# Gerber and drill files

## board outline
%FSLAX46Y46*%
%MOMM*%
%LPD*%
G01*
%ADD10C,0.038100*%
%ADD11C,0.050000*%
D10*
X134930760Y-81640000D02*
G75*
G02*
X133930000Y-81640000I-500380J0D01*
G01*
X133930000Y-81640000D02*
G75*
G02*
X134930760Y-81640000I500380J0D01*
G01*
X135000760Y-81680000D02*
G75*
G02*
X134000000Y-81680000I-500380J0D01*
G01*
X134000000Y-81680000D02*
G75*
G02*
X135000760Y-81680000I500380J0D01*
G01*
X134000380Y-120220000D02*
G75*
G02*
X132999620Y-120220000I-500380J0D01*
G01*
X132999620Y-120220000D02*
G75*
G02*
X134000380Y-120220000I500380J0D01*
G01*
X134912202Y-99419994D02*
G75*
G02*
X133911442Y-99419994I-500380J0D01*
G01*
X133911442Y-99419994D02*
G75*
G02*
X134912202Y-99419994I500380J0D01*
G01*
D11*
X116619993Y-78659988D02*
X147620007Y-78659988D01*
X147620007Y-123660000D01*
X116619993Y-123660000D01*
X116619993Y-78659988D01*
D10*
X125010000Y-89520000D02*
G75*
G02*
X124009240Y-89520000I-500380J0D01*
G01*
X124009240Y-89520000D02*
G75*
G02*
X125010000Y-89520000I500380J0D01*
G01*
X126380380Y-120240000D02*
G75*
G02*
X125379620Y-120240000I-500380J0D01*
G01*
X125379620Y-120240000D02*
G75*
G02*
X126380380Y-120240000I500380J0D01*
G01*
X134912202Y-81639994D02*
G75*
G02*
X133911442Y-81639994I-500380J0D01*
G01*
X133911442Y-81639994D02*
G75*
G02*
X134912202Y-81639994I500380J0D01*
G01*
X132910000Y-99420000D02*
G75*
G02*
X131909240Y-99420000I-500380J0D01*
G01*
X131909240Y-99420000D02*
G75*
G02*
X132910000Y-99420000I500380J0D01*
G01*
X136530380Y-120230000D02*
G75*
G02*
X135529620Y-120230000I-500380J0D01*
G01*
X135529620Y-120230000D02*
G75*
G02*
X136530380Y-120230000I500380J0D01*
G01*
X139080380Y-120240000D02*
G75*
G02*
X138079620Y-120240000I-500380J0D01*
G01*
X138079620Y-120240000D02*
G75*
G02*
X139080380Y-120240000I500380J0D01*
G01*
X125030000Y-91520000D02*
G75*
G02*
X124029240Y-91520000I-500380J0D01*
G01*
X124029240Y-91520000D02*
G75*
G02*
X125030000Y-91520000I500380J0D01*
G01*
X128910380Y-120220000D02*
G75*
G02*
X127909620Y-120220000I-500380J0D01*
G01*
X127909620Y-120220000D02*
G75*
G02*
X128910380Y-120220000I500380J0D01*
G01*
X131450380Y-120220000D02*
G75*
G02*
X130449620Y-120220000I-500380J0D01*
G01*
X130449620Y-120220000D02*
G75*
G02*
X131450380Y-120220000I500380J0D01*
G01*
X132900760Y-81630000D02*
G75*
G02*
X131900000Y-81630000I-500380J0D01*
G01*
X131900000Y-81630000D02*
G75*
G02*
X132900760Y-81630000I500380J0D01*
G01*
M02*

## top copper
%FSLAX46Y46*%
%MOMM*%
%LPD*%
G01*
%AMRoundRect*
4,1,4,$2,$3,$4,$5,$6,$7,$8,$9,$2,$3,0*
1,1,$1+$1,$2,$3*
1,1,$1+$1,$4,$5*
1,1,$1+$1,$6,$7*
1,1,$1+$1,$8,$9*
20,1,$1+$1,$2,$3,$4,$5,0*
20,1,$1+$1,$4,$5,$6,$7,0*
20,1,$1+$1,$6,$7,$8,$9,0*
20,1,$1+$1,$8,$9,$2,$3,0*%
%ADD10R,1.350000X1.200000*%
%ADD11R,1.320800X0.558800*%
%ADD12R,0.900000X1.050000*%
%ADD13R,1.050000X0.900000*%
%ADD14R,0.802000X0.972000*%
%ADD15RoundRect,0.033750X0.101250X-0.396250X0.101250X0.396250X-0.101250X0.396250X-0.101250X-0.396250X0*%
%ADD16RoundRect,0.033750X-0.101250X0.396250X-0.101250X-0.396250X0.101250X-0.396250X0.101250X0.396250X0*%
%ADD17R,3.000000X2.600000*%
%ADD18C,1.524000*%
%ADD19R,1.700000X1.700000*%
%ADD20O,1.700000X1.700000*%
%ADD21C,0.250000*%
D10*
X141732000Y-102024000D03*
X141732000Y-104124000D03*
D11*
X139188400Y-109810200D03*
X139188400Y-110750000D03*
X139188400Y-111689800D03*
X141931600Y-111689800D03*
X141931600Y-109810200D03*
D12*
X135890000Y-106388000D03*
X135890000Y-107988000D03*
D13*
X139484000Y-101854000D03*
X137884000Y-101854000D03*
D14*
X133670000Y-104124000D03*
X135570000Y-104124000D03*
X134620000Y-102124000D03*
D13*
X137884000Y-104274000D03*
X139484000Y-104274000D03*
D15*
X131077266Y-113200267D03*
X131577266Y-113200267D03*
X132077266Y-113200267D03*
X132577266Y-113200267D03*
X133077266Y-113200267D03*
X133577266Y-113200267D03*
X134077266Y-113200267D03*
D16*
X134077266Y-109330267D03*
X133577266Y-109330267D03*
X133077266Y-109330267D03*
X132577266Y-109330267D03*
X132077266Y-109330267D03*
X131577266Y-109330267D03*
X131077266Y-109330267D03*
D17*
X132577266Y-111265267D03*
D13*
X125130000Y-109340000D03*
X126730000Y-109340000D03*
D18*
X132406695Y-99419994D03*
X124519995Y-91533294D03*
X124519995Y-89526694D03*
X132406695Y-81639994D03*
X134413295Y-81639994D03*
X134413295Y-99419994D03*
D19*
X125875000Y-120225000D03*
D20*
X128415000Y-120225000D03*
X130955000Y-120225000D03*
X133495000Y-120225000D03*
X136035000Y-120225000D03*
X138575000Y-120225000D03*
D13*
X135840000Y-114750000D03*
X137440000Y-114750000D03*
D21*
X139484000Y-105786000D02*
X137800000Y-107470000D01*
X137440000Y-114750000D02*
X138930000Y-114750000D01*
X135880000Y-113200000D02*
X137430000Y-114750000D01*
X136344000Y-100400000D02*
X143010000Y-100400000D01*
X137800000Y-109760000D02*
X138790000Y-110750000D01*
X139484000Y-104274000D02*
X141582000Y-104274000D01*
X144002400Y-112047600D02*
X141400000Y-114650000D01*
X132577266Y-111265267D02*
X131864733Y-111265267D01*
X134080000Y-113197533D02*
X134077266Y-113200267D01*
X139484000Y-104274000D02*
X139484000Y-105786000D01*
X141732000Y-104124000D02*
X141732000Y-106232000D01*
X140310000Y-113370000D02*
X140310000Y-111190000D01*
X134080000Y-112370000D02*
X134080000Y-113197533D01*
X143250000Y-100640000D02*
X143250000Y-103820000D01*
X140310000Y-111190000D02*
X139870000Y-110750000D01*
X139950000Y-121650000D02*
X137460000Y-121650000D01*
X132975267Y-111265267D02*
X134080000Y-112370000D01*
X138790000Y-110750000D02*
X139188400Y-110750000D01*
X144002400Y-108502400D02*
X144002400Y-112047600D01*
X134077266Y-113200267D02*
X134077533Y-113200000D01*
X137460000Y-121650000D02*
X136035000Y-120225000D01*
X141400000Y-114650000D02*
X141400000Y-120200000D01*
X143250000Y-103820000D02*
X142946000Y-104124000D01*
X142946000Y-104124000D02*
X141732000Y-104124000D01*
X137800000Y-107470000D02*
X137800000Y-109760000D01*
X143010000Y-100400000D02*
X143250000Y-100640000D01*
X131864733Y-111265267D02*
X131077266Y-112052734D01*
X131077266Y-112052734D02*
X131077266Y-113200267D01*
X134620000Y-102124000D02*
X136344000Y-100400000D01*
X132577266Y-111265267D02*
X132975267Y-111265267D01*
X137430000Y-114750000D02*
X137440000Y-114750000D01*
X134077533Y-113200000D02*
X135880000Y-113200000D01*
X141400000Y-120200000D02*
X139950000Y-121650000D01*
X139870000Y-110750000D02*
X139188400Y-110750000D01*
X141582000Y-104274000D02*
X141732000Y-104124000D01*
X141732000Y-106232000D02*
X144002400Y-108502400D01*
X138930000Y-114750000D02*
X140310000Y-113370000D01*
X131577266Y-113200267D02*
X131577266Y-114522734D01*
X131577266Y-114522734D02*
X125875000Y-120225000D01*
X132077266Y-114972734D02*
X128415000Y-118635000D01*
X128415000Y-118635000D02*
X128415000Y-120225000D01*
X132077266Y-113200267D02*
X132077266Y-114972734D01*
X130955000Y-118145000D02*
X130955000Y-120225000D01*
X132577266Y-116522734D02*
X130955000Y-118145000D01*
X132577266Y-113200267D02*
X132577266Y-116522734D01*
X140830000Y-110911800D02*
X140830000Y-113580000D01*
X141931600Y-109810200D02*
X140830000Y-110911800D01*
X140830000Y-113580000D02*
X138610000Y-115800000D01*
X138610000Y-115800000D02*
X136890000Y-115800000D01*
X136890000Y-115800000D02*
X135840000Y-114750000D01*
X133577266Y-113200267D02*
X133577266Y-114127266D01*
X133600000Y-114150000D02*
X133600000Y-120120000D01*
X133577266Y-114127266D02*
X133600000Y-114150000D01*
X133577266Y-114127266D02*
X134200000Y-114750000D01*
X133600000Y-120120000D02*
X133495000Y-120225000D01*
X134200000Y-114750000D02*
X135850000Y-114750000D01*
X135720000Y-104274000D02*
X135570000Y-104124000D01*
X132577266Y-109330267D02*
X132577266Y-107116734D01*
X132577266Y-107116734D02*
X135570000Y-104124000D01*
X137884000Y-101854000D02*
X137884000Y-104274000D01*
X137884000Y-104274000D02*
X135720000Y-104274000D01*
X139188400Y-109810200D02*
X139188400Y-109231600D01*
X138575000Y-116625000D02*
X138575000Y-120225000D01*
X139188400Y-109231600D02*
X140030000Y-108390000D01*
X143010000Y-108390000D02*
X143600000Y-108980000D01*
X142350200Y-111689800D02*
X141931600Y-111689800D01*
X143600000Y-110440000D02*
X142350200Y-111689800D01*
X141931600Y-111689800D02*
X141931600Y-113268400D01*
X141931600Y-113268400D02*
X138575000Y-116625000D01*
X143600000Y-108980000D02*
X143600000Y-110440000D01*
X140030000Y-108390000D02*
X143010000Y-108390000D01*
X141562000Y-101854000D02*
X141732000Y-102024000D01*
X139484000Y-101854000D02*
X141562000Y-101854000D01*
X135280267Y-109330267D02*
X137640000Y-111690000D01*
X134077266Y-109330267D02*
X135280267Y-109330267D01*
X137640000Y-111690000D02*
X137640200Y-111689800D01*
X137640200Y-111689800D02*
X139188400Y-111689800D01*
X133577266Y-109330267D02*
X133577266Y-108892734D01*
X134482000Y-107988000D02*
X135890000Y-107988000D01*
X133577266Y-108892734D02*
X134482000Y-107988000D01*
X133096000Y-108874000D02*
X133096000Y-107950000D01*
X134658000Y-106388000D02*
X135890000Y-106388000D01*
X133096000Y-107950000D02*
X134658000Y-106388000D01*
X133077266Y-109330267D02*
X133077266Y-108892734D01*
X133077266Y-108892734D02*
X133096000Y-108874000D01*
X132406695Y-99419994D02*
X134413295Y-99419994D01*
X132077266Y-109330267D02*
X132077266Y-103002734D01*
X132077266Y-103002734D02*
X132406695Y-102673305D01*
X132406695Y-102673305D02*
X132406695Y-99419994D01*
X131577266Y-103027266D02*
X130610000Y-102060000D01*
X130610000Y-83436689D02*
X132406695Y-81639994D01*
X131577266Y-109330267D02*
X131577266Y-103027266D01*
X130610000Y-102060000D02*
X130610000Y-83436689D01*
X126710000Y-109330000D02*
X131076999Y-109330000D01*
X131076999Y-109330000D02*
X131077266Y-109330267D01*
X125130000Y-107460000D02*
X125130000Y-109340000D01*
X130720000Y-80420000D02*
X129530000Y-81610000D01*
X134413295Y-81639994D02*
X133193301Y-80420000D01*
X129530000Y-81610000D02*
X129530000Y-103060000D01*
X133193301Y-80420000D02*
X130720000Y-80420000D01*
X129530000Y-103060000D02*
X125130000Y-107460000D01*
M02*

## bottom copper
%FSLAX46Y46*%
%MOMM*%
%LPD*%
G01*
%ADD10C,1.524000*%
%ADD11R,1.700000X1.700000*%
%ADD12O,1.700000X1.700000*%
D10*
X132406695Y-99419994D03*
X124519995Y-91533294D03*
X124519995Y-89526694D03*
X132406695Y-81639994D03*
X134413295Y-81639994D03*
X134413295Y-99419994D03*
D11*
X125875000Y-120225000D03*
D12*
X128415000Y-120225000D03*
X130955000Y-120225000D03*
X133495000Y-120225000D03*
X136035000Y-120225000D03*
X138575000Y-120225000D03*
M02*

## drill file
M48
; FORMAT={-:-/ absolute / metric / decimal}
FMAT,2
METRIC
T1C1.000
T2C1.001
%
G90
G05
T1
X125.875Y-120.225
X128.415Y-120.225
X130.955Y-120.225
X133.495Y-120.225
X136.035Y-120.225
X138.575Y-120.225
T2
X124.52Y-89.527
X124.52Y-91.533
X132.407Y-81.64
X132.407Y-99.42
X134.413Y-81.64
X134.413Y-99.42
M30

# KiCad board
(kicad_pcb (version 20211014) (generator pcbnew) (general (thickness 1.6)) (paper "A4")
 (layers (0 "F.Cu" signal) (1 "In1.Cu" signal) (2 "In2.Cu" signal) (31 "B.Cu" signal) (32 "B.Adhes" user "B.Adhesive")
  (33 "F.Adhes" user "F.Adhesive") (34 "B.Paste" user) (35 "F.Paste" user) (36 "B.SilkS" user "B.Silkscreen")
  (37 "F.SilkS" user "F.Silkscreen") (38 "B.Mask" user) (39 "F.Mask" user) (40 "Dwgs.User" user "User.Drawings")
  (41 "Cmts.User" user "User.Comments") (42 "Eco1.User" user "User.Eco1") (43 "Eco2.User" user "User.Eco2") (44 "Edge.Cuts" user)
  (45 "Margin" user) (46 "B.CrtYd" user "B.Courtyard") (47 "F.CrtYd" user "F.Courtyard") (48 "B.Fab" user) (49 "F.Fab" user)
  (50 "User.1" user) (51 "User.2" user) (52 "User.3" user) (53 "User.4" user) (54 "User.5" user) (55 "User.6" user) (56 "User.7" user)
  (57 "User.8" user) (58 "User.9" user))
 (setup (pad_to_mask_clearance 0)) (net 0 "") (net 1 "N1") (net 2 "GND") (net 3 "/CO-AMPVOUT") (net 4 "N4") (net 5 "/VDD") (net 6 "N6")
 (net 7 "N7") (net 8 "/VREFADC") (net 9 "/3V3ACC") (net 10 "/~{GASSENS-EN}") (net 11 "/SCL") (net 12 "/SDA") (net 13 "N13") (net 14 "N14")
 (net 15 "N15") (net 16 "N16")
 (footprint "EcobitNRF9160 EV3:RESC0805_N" (layer "F.Cu") (at 141.732 103.124 -90)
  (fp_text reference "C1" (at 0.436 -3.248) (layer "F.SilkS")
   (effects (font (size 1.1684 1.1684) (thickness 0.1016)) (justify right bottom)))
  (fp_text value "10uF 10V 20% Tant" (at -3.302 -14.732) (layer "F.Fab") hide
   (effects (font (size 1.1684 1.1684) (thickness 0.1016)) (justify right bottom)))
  (pad "1" smd rect (at -1.1 0 270) (size 1.2 1.35) (layers "F.Cu" "F.Paste" "F.Mask") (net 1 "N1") (solder_mask_margin 0.1016))
  (pad "2" smd rect (at 1 0 270) (size 1.2 1.35) (layers "F.Cu" "F.Paste" "F.Mask") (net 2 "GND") (solder_mask_margin 0.1016)))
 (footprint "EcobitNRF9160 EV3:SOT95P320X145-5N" (layer "F.Cu") (at 140.56 110.75)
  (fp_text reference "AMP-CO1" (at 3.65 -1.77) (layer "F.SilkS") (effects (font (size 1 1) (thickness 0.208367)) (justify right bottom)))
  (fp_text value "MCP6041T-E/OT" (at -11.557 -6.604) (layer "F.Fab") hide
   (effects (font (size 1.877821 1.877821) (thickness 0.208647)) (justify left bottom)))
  (pad "1" smd rect (at -1.3716 -0.9398) (size 1.3208 0.5588) (layers "F.Cu" "F.Paste" "F.Mask") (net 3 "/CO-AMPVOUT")
   (solder_mask_margin 0.1016))
  (pad "2" smd rect (at -1.3716 0) (size 1.3208 0.5588) (layers "F.Cu" "F.Paste" "F.Mask") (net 2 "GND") (solder_mask_margin 0.1016))
  (pad "3" smd rect (at -1.3716 0.9398) (size 1.3208 0.5588) (layers "F.Cu" "F.Paste" "F.Mask") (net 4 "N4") (solder_mask_margin 0.1016))
  (pad "4" smd rect (at 1.3716 0.9398) (size 1.3208 0.5588) (layers "F.Cu" "F.Paste" "F.Mask") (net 3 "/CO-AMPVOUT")
   (solder_mask_margin 0.1016))
  (pad "5" smd rect (at 1.3716 -0.9398) (size 1.3208 0.5588) (layers "F.Cu" "F.Paste" "F.Mask") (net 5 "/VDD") (solder_mask_margin 0.1016)))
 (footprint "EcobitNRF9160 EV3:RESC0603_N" (layer "F.Cu") (at 135.89 107.188 -90)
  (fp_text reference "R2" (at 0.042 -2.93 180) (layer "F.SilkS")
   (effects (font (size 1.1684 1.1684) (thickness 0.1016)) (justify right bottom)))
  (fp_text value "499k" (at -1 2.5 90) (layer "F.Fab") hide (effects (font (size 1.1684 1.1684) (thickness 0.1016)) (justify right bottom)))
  (pad "1" smd rect (at -0.8 0 270) (size 1.05 0.9) (layers "F.Cu" "F.Paste" "F.Mask") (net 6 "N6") (solder_mask_margin 0.1016))
  (pad "2" smd rect (at 0.8 0 270) (size 1.05 0.9) (layers "F.Cu" "F.Paste" "F.Mask") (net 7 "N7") (solder_mask_margin 0.1016)))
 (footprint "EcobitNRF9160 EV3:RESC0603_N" (layer "F.Cu") (at 138.684 101.854 180)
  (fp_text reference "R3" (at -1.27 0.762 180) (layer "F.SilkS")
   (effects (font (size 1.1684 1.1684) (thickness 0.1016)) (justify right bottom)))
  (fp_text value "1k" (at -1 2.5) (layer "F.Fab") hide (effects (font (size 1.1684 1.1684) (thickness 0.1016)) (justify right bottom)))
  (pad "1" smd rect (at -0.8 0 180) (size 1.05 0.9) (layers "F.Cu" "F.Paste" "F.Mask") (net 1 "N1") (solder_mask_margin 0.1016))
  (pad "2" smd rect (at 0.8 0 180) (size 1.05 0.9) (layers "F.Cu" "F.Paste" "F.Mask") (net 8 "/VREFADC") (solder_mask_margin 0.1016)))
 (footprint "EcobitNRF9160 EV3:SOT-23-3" (layer "F.Cu") (at 134.62 103.124)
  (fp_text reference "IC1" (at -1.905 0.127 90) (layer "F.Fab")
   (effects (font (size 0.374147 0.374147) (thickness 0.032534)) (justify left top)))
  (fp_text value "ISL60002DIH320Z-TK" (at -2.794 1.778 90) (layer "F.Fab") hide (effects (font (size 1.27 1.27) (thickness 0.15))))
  (pad "1" smd rect (at -0.95 1 90) (size 0.972 0.802) (layers "F.Cu" "F.Paste" "F.Mask") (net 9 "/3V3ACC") (solder_mask_margin 0.1016))
  (pad "2" smd rect (at 0.95 1 90) (size 0.972 0.802) (layers "F.Cu" "F.Paste" "F.Mask") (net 8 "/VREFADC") (solder_mask_margin 0.1016))
  (pad "3" smd rect (at 0 -1 90) (size 0.972 0.802) (layers "F.Cu" "F.Paste" "F.Mask") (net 2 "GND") (solder_mask_margin 0.1016)))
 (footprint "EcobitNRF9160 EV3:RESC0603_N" (layer "F.Cu") (at 138.684 104.274)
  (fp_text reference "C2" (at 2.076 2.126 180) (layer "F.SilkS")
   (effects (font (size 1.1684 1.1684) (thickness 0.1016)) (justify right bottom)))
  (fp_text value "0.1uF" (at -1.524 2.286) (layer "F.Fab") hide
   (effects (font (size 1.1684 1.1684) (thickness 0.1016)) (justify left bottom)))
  (pad "1" smd rect (at -0.8 0) (size 1.05 0.9) (layers "F.Cu" "F.Paste" "F.Mask") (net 8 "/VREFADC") (solder_mask_margin 0.1016))
  (pad "2" smd rect (at 0.8 0) (size 1.05 0.9) (layers "F.Cu" "F.Paste" "F.Mask") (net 2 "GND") (solder_mask_margin 0.1016)))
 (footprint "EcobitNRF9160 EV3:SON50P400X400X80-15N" (layer "F.Cu") (at 132.577266 111.265267 90)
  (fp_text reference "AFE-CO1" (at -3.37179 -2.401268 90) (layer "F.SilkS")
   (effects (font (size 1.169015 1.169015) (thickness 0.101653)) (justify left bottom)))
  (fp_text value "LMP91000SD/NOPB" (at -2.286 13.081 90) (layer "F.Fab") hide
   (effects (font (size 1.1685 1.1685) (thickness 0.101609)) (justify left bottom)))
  (pad "1" smd roundrect (at -1.935 -1.5 90) (size 0.86 0.27) (layers "F.Cu" "F.Paste" "F.Mask") (roundrect_rratio 0.125) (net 2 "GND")
   (solder_mask_margin 0.1016))
  (pad "2" smd roundrect (at -1.935 -1 90) (size 0.86 0.27) (layers "F.Cu" "F.Paste" "F.Mask") (roundrect_rratio 0.125)
   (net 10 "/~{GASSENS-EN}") (solder_mask_margin 0.1016))
  (pad "3" smd roundrect (at -1.935 -0.5 90) (size 0.86 0.27) (layers "F.Cu" "F.Paste" "F.Mask") (roundrect_rratio 0.125) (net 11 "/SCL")
   (solder_mask_margin 0.1016))
  (pad "4" smd roundrect (at -1.935 0 90) (size 0.86 0.27) (layers "F.Cu" "F.Paste" "F.Mask") (roundrect_rratio 0.125) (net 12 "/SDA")
   (solder_mask_margin 0.1016))
  (pad "5" smd roundrect (at -1.935 0.5 90) (size 0.86 0.27) (layers "F.Cu" "F.Paste" "F.Mask") (roundrect_rratio 0.125)
   (solder_mask_margin 0.1016))
  (pad "6" smd roundrect (at -1.935 1 90) (size 0.86 0.27) (layers "F.Cu" "F.Paste" "F.Mask") (roundrect_rratio 0.125) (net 5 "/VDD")
   (solder_mask_margin 0.1016))
  (pad "7" smd roundrect (at -1.935 1.5 90) (size 0.86 0.27) (layers "F.Cu" "F.Paste" "F.Mask") (roundrect_rratio 0.125) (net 2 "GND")
   (solder_mask_margin 0.1016))
  (pad "8" smd roundrect (at 1.935 1.5 270) (size 0.86 0.27) (layers "F.Cu" "F.Paste" "F.Mask") (roundrect_rratio 0.125) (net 4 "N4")
   (solder_mask_margin 0.1016))
  (pad "9" smd roundrect (at 1.935 1 270) (size 0.86 0.27) (layers "F.Cu" "F.Paste" "F.Mask") (roundrect_rratio 0.125) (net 7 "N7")
   (solder_mask_margin 0.1016))
  (pad "10" smd roundrect (at 1.935 0.5 270) (size 0.86 0.27) (layers "F.Cu" "F.Paste" "F.Mask") (roundrect_rratio 0.125) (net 6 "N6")
   (solder_mask_margin 0.1016))
  (pad "11" smd roundrect (at 1.935 0 270) (size 0.86 0.27) (layers "F.Cu" "F.Paste" "F.Mask") (roundrect_rratio 0.125) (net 8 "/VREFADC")
   (solder_mask_margin 0.1016))
  (pad "12" smd roundrect (at 1.935 -0.5 270) (size 0.86 0.27) (layers "F.Cu" "F.Paste" "F.Mask") (roundrect_rratio 0.125) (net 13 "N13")
   (solder_mask_margin 0.1016))
  (pad "13" smd roundrect (at 1.935 -1 270) (size 0.86 0.27) (layers "F.Cu" "F.Paste" "F.Mask") (roundrect_rratio 0.125) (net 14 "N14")
   (solder_mask_margin 0.1016))
  (pad "14" smd roundrect (at 1.935 -1.5 270) (size 0.86 0.27) (layers "F.Cu" "F.Paste" "F.Mask") (roundrect_rratio 0.125) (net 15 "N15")
   (solder_mask_margin 0.1016))
  (pad "15" smd rect (at 0 0 90) (size 2.6 3) (layers "F.Cu" "F.Mask") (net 2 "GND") (solder_mask_margin 0.1016)))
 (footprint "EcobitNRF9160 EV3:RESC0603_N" (layer "F.Cu") (at 125.93 109.34)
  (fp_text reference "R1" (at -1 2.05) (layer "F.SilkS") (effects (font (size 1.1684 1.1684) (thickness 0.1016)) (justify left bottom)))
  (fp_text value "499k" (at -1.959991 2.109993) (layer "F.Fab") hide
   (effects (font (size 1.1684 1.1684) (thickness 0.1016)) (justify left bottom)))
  (pad "1" smd rect (at -0.8 0) (size 1.05 0.9) (layers "F.Cu" "F.Paste" "F.Mask") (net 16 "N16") (solder_mask_margin 0.1016))
  (pad "2" smd rect (at 0.8 0) (size 1.05 0.9) (layers "F.Cu" "F.Paste" "F.Mask") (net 15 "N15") (solder_mask_margin 0.1016)))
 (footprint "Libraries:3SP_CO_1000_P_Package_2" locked (layer "F.Cu") (at 133.409995 90.529994)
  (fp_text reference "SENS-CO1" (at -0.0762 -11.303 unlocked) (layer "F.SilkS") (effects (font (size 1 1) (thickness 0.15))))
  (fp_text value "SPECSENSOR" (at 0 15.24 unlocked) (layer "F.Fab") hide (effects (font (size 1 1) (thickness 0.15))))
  (pad "1" thru_hole circle locked (at -1.0033 8.89) (size 1.524 1.524) (drill 1.00076) (layers *.Cu *.Mask) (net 13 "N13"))
  (pad "2" thru_hole circle locked (at -8.89 1.0033) (size 1.524 1.524) (drill 1.00076) (layers *.Cu *.Mask))
  (pad "3" thru_hole circle locked (at -8.89 -1.0033) (size 1.524 1.524) (drill 1.00076) (layers *.Cu *.Mask))
  (pad "4" thru_hole circle locked (at -1.0033 -8.89) (size 1.524 1.524) (drill 1.00076) (layers *.Cu *.Mask) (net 14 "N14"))
  (pad "5" thru_hole circle locked (at 1.0033 -8.89) (size 1.524 1.524) (drill 1.00076) (layers *.Cu *.Mask) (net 16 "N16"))
  (pad "6" thru_hole circle locked (at 1.0033 8.89) (size 1.524 1.524) (drill 1.00076) (layers *.Cu *.Mask) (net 13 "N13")))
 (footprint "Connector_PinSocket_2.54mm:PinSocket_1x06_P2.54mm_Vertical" (layer "F.Cu") (at 125.875 120.225 90)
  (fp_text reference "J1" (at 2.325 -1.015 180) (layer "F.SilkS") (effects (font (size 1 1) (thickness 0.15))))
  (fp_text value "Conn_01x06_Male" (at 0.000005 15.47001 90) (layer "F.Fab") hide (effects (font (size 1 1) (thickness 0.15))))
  (pad "1" thru_hole rect (at 0 0 90) (size 1.7 1.7) (drill 1) (layers *.Cu *.Mask) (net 10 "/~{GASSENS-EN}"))
  (pad "2" thru_hole oval (at 0 2.54 90) (size 1.7 1.7) (drill 1) (layers *.Cu *.Mask) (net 11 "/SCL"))
  (pad "3" thru_hole oval (at 0 5.08 90) (size 1.7 1.7) (drill 1) (layers *.Cu *.Mask) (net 12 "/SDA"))
  (pad "4" thru_hole oval (at 0 7.62 90) (size 1.7 1.7) (drill 1) (layers *.Cu *.Mask) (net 5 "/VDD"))
  (pad "5" thru_hole oval (at 0 10.16 90) (size 1.7 1.7) (drill 1) (layers *.Cu *.Mask) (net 2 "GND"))
  (pad "6" thru_hole oval (at 0 12.7 90) (size 1.7 1.7) (drill 1) (layers *.Cu *.Mask) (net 3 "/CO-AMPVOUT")))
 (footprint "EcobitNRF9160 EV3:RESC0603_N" (layer "F.Cu") (at 136.64 114.75)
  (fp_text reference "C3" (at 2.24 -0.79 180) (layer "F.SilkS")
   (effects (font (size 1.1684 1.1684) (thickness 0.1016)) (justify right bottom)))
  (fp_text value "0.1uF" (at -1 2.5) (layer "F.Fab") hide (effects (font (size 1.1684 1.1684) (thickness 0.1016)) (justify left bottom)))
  (pad "1" smd rect (at -0.8 0) (size 1.05 0.9) (layers "F.Cu" "F.Paste" "F.Mask") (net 5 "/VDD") (solder_mask_margin 0.1016))
  (pad "2" smd rect (at 0.8 0) (size 1.05 0.9) (layers "F.Cu" "F.Paste" "F.Mask") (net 2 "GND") (solder_mask_margin 0.1016)))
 (gr_circle (center 134.43038 81.64) (end 134.93076 81.64) (layer "Edge.Cuts") (width 0.0381) (fill none))
 (gr_circle (center 134.50038 81.68) (end 135.00076 81.68) (layer "Edge.Cuts") (width 0.0381) (fill none))
 (gr_circle (center 133.5 120.22) (end 134.00038 120.22) (layer "Edge.Cuts") (width 0.0381) (fill none))
 (gr_circle (center 134.411822 99.419994) (end 134.912202 99.419994) (layer "Edge.Cuts") (width 0.0381) (fill none))
 (gr_rect (start 116.619993 78.659988) (end 147.620007 123.66) (layer "Edge.Cuts") (width 0.05) (fill none))
 (gr_circle (center 124.50962 89.52) (end 125.01 89.52) (layer "Edge.Cuts") (width 0.0381) (fill none))
 (gr_circle (center 125.88 120.24) (end 126.38038 120.24) (layer "Edge.Cuts") (width 0.0381) (fill none))
 (gr_circle (center 134.411822 81.639994) (end 134.912202 81.639994) (layer "Edge.Cuts") (width 0.0381) (fill none))
 (gr_circle (center 132.40962 99.42) (end 132.91 99.42) (layer "Edge.Cuts") (width 0.0381) (fill none))
 (gr_circle (center 136.03 120.23) (end 136.53038 120.23) (layer "Edge.Cuts") (width 0.0381) (fill none))
 (gr_circle (center 138.58 120.24) (end 139.08038 120.24) (layer "Edge.Cuts") (width 0.0381) (fill none))
 (gr_circle (center 124.52962 91.52) (end 125.03 91.52) (layer "Edge.Cuts") (width 0.0381) (fill none))
 (gr_circle (center 128.41 120.22) (end 128.91038 120.22) (layer "Edge.Cuts") (width 0.0381) (fill none))
 (gr_circle (center 130.95 120.22) (end 131.45038 120.22) (layer "Edge.Cuts") (width 0.0381) (fill none))
 (gr_circle (center 132.40038 81.63) (end 132.90076 81.63) (layer "Edge.Cuts") (width 0.0381) (fill none))
 (segment (start 139.484 105.786) (end 137.8 107.47) (width 0.25) (layer "F.Cu") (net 2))
 (segment (start 137.44 114.75) (end 138.93 114.75) (width 0.25) (layer "F.Cu") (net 2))
 (segment (start 135.88 113.2) (end 137.43 114.75) (width 0.25) (layer "F.Cu") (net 2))
 (segment (start 136.344 100.4) (end 143.01 100.4) (width 0.25) (layer "F.Cu") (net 2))
 (segment (start 137.8 109.76) (end 138.79 110.75) (width 0.25) (layer "F.Cu") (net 2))
 (segment (start 139.484 104.274) (end 141.582 104.274) (width 0.25) (layer "F.Cu") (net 2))
 (segment (start 144.0024 112.0476) (end 141.4 114.65) (width 0.25) (layer "F.Cu") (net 2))
 (segment (start 132.577266 111.265267) (end 131.864733 111.265267) (width 0.25) (layer "F.Cu") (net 2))
 (segment (start 134.08 113.197533) (end 134.077266 113.200267) (width 0.25) (layer "F.Cu") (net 2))
 (segment (start 139.484 104.274) (end 139.484 105.786) (width 0.25) (layer "F.Cu") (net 2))
 (segment (start 141.732 104.124) (end 141.732 106.232) (width 0.25) (layer "F.Cu") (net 2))
 (segment (start 140.31 113.37) (end 140.31 111.19) (width 0.25) (layer "F.Cu") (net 2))
 (segment (start 134.08 112.37) (end 134.08 113.197533) (width 0.25) (layer "F.Cu") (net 2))
 (segment (start 143.25 100.64) (end 143.25 103.82) (width 0.25) (layer "F.Cu") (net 2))
 (segment (start 140.31 111.19) (end 139.87 110.75) (width 0.25) (layer "F.Cu") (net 2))
 (segment (start 139.95 121.65) (end 137.46 121.65) (width 0.25) (layer "F.Cu") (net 2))
 (segment (start 132.975267 111.265267) (end 134.08 112.37) (width 0.25) (layer "F.Cu") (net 2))
 (segment (start 138.79 110.75) (end 139.1884 110.75) (width 0.25) (layer "F.Cu") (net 2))
 (segment (start 144.0024 108.5024) (end 144.0024 112.0476) (width 0.25) (layer "F.Cu") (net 2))
 (segment (start 134.077266 113.200267) (end 134.077533 113.2) (width 0.25) (layer "F.Cu") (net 2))
 (segment (start 137.46 121.65) (end 136.035 120.225) (width 0.25) (layer "F.Cu") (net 2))
 (segment (start 141.4 114.65) (end 141.4 120.2) (width 0.25) (layer "F.Cu") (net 2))
 (segment (start 143.25 103.82) (end 142.946 104.124) (width 0.25) (layer "F.Cu") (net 2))
 (segment (start 142.946 104.124) (end 141.732 104.124) (width 0.25) (layer "F.Cu") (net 2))
 (segment (start 137.8 107.47) (end 137.8 109.76) (width 0.25) (layer "F.Cu") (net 2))
 (segment (start 143.01 100.4) (end 143.25 100.64) (width 0.25) (layer "F.Cu") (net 2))
 (segment (start 131.864733 111.265267) (end 131.077266 112.052734) (width 0.25) (layer "F.Cu") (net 2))
 (segment (start 131.077266 112.052734) (end 131.077266 113.200267) (width 0.25) (layer "F.Cu") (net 2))
 (segment (start 134.62 102.124) (end 136.344 100.4) (width 0.25) (layer "F.Cu") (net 2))
 (segment (start 132.577266 111.265267) (end 132.975267 111.265267) (width 0.25) (layer "F.Cu") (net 2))
 (segment (start 137.43 114.75) (end 137.44 114.75) (width 0.25) (layer "F.Cu") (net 2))
 (segment (start 134.077533 113.2) (end 135.88 113.2) (width 0.25) (layer "F.Cu") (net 2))
 (segment (start 141.4 120.2) (end 139.95 121.65) (width 0.25) (layer "F.Cu") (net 2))
 (segment (start 139.87 110.75) (end 139.1884 110.75) (width 0.25) (layer "F.Cu") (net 2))
 (segment (start 141.582 104.274) (end 141.732 104.124) (width 0.25) (layer "F.Cu") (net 2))
 (segment (start 141.732 106.232) (end 144.0024 108.5024) (width 0.25) (layer "F.Cu") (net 2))
 (segment (start 138.93 114.75) (end 140.31 113.37) (width 0.25) (layer "F.Cu") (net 2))
 (segment (start 131.577266 113.200267) (end 131.577266 114.522734) (width 0.25) (layer "F.Cu") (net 10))
 (segment (start 131.577266 114.522734) (end 125.875 120.225) (width 0.25) (layer "F.Cu") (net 10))
 (segment (start 132.077266 114.972734) (end 128.415 118.635) (width 0.25) (layer "F.Cu") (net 11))
 (segment (start 128.415 118.635) (end 128.415 120.225) (width 0.25) (layer "F.Cu") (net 11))
 (segment (start 132.077266 113.200267) (end 132.077266 114.972734) (width 0.25) (layer "F.Cu") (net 11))
 (segment (start 130.955 118.145) (end 130.955 120.225) (width 0.25) (layer "F.Cu") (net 12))
 (segment (start 132.577266 116.522734) (end 130.955 118.145) (width 0.25) (layer "F.Cu") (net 12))
 (segment (start 132.577266 113.200267) (end 132.577266 116.522734) (width 0.25) (layer "F.Cu") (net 12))
 (segment (start 140.83 110.9118) (end 140.83 113.58) (width 0.25) (layer "F.Cu") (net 5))
 (segment (start 141.9316 109.8102) (end 140.83 110.9118) (width 0.25) (layer "F.Cu") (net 5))
 (segment (start 140.83 113.58) (end 138.61 115.8) (width 0.25) (layer "F.Cu") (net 5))
 (segment (start 138.61 115.8) (end 136.89 115.8) (width 0.25) (layer "F.Cu") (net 5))
 (segment (start 136.89 115.8) (end 135.84 114.75) (width 0.25) (layer "F.Cu") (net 5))
 (segment (start 133.577266 113.200267) (end 133.577266 114.127266) (width 0.25) (layer "F.Cu") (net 5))
 (segment (start 133.6 114.15) (end 133.6 120.12) (width 0.25) (layer "F.Cu") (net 5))
 (segment (start 133.577266 114.127266) (end 133.6 114.15) (width 0.25) (layer "F.Cu") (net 5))
 (segment (start 133.577266 114.127266) (end 134.2 114.75) (width 0.25) (layer "F.Cu") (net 5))
 (segment (start 133.6 120.12) (end 133.495 120.225) (width 0.25) (layer "F.Cu") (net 5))
 (segment (start 134.2 114.75) (end 135.85 114.75) (width 0.25) (layer "F.Cu") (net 5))
 (segment (start 135.72 104.274) (end 135.57 104.124) (width 0.25) (layer "F.Cu") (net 8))
 (segment (start 132.577266 109.330267) (end 132.577266 107.116734) (width 0.25) (layer "F.Cu") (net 8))
 (segment (start 132.577266 107.116734) (end 135.57 104.124) (width 0.25) (layer "F.Cu") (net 8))
 (segment (start 137.884 101.854) (end 137.884 104.274) (width 0.25) (layer "F.Cu") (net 8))
 (segment (start 137.884 104.274) (end 135.72 104.274) (width 0.25) (layer "F.Cu") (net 8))
 (segment (start 139.1884 109.8102) (end 139.1884 109.2316) (width 0.25) (layer "F.Cu") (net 3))
 (segment (start 138.575 116.625) (end 138.575 120.225) (width 0.25) (layer "F.Cu") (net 3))
 (segment (start 139.1884 109.2316) (end 140.03 108.39) (width 0.25) (layer "F.Cu") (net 3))
 (segment (start 143.01 108.39) (end 143.6 108.98) (width 0.25) (layer "F.Cu") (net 3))
 (segment (start 142.3502 111.6898) (end 141.9316 111.6898) (width 0.25) (layer "F.Cu") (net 3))
 (segment (start 143.6 110.44) (end 142.3502 111.6898) (width 0.25) (layer "F.Cu") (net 3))
 (segment (start 141.9316 111.6898) (end 141.9316 113.2684) (width 0.25) (layer "F.Cu") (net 3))
 (segment (start 141.9316 113.2684) (end 138.575 116.625) (width 0.25) (layer "F.Cu") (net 3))
 (segment (start 143.6 108.98) (end 143.6 110.44) (width 0.25) (layer "F.Cu") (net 3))
 (segment (start 140.03 108.39) (end 143.01 108.39) (width 0.25) (layer "F.Cu") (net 3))
 (segment (start 141.562 101.854) (end 141.732 102.024) (width 0.25) (layer "F.Cu") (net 1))
 (segment (start 139.484 101.854) (end 141.562 101.854) (width 0.25) (layer "F.Cu") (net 1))
 (segment (start 135.280267 109.330267) (end 137.64 111.69) (width 0.25) (layer "F.Cu") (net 4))
 (segment (start 134.077266 109.330267) (end 135.280267 109.330267) (width 0.25) (layer "F.Cu") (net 4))
 (segment (start 137.64 111.69) (end 137.6402 111.6898) (width 0.25) (layer "F.Cu") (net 4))
 (segment (start 137.6402 111.6898) (end 139.1884 111.6898) (width 0.25) (layer "F.Cu") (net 4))
 (segment (start 133.577266 109.330267) (end 133.577266 108.892734) (width 0.25) (layer "F.Cu") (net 7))
 (segment (start 134.482 107.988) (end 135.89 107.988) (width 0.25) (layer "F.Cu") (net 7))
 (segment (start 133.577266 108.892734) (end 134.482 107.988) (width 0.25) (layer "F.Cu") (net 7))
 (segment (start 133.096 108.874) (end 133.096 107.95) (width 0.25) (layer "F.Cu") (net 6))
 (segment (start 134.658 106.388) (end 135.89 106.388) (width 0.25) (layer "F.Cu") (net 6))
 (segment (start 133.096 107.95) (end 134.658 106.388) (width 0.25) (layer "F.Cu") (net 6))
 (segment (start 133.077266 109.330267) (end 133.077266 108.892734) (width 0.25) (layer "F.Cu") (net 6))
 (segment (start 133.077266 108.892734) (end 133.096 108.874) (width 0.25) (layer "F.Cu") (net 6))
 (segment (start 132.406695 99.419994) (end 134.413295 99.419994) (width 0.25) (layer "F.Cu") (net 13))
 (segment (start 132.077266 109.330267) (end 132.077266 103.002734) (width 0.25) (layer "F.Cu") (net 13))
 (segment (start 132.077266 103.002734) (end 132.406695 102.673305) (width 0.25) (layer "F.Cu") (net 13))
 (segment (start 132.406695 102.673305) (end 132.406695 99.419994) (width 0.25) (layer "F.Cu") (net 13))
 (segment (start 131.577266 103.027266) (end 130.61 102.06) (width 0.25) (layer "F.Cu") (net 14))
 (segment (start 130.61 83.436689) (end 132.406695 81.639994) (width 0.25) (layer "F.Cu") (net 14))
 (segment (start 131.577266 109.330267) (end 131.577266 103.027266) (width 0.25) (layer "F.Cu") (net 14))
 (segment (start 130.61 102.06) (end 130.61 83.436689) (width 0.25) (layer "F.Cu") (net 14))
 (segment (start 126.71 109.33) (end 131.076999 109.33) (width 0.25) (layer "F.Cu") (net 15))
 (segment (start 131.076999 109.33) (end 131.077266 109.330267) (width 0.25) (layer "F.Cu") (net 15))
 (segment (start 125.13 107.46) (end 125.13 109.34) (width 0.25) (layer "F.Cu") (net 16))
 (segment (start 130.72 80.42) (end 129.53 81.61) (width 0.25) (layer "F.Cu") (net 16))
 (segment (start 134.413295 81.639994) (end 133.193301 80.42) (width 0.25) (layer "F.Cu") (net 16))
 (segment (start 129.53 81.61) (end 129.53 103.06) (width 0.25) (layer "F.Cu") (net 16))
 (segment (start 133.193301 80.42) (end 130.72 80.42) (width 0.25) (layer "F.Cu") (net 16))
 (segment (start 129.53 103.06) (end 125.13 107.46) (width 0.25) (layer "F.Cu") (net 16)))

